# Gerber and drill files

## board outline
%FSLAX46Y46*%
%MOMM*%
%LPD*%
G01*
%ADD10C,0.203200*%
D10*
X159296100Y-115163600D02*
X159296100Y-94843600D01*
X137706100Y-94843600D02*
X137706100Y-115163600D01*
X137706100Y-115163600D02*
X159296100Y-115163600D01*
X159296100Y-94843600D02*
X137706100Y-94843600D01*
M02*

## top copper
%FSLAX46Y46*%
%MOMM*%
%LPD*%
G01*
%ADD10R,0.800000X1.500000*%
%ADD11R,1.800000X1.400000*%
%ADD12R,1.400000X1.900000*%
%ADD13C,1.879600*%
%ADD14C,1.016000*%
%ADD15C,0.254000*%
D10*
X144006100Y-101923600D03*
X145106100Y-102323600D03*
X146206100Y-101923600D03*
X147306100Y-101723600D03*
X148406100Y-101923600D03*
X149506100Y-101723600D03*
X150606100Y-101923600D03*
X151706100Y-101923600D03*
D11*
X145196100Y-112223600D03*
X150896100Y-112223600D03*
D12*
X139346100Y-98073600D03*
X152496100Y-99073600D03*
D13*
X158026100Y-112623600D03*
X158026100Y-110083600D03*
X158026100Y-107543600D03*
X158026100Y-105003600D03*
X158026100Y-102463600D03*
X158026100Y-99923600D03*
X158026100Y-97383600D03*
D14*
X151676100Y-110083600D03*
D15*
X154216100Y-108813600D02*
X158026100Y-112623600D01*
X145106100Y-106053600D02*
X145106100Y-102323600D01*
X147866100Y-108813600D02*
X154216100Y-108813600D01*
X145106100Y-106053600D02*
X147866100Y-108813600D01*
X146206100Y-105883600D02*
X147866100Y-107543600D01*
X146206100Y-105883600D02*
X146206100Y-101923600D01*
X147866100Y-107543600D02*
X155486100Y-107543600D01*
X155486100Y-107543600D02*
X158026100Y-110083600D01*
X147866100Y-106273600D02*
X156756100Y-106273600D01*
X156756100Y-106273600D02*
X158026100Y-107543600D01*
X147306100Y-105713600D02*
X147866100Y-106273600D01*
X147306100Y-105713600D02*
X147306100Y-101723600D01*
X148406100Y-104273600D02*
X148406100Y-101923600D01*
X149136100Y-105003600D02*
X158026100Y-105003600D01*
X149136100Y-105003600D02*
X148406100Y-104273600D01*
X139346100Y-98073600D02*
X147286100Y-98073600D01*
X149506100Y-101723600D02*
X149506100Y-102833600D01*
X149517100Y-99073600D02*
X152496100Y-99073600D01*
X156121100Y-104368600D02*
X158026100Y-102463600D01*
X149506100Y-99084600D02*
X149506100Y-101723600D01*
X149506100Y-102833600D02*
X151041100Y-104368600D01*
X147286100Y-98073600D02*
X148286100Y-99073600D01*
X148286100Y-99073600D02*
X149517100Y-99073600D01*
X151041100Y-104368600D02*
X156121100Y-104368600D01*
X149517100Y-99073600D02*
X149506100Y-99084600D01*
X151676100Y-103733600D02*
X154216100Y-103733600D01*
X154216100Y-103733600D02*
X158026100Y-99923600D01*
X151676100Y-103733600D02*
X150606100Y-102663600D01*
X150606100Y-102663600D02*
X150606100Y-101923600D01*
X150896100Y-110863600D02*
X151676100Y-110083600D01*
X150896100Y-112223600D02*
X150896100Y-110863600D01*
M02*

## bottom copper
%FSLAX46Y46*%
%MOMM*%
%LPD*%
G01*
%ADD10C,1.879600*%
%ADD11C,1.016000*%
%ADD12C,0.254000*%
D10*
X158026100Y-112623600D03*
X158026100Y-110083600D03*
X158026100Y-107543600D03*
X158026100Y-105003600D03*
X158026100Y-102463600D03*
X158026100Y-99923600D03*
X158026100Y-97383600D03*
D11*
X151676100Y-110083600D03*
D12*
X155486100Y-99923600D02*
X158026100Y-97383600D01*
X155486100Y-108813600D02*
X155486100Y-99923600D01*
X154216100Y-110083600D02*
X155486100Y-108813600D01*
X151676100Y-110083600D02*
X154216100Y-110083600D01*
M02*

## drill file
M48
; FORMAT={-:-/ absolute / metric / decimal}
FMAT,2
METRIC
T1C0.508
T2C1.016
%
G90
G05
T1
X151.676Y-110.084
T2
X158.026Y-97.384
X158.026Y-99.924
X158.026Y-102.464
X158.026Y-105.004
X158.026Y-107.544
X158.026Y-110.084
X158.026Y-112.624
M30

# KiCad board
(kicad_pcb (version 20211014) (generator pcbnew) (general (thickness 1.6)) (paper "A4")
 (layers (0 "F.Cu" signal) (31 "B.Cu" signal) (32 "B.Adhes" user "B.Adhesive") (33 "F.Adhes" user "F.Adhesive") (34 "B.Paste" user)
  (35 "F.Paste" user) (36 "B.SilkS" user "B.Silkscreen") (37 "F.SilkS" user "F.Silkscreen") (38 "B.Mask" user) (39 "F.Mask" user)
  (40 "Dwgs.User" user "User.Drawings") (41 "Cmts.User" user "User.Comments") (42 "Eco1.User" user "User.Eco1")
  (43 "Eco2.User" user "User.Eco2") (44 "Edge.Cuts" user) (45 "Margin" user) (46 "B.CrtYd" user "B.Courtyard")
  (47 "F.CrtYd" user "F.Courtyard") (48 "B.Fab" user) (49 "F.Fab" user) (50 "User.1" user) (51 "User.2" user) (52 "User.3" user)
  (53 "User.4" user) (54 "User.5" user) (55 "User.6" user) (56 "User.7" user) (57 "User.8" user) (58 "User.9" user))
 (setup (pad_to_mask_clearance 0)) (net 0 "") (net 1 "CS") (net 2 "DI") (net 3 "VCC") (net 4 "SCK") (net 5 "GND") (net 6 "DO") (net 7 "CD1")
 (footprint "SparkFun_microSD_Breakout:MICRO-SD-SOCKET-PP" (layer "F.Cu") (at 152.9461 112.6236)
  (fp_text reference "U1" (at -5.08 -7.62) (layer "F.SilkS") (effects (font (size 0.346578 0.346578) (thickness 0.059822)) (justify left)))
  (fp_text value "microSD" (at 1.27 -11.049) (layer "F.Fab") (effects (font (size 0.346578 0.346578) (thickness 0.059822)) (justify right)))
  (pad "1" smd rect (at -8.94 -10.7) (size 0.8 1.5) (layers "F.Cu" "F.Paste" "F.Mask") (solder_mask_margin 0.1016))
  (pad "2" smd rect (at -7.84 -10.3) (size 0.8 1.5) (layers "F.Cu" "F.Paste" "F.Mask") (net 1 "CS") (solder_mask_margin 0.1016))
  (pad "3" smd rect (at -6.74 -10.7) (size 0.8 1.5) (layers "F.Cu" "F.Paste" "F.Mask") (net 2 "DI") (solder_mask_margin 0.1016))
  (pad "4" smd rect (at -5.64 -10.9) (size 0.8 1.5) (layers "F.Cu" "F.Paste" "F.Mask") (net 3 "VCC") (solder_mask_margin 0.1016))
  (pad "5" smd rect (at -4.54 -10.7) (size 0.8 1.5) (layers "F.Cu" "F.Paste" "F.Mask") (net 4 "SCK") (solder_mask_margin 0.1016))
  (pad "6" smd rect (at -3.44 -10.9) (size 0.8 1.5) (layers "F.Cu" "F.Paste" "F.Mask") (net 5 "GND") (solder_mask_margin 0.1016))
  (pad "7" smd rect (at -2.34 -10.7) (size 0.8 1.5) (layers "F.Cu" "F.Paste" "F.Mask") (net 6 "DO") (solder_mask_margin 0.1016))
  (pad "8" smd rect (at -1.24 -10.7) (size 0.8 1.5) (layers "F.Cu" "F.Paste" "F.Mask") (solder_mask_margin 0.1016))
  (pad "CD1" smd rect (at -7.75 -0.4) (size 1.8 1.4) (layers "F.Cu" "F.Paste" "F.Mask") (solder_mask_margin 0.1016))
  (pad "CD2" smd rect (at -2.05 -0.4) (size 1.8 1.4) (layers "F.Cu" "F.Paste" "F.Mask") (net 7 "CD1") (solder_mask_margin 0.1016))
  (pad "GND1" smd rect (at -13.6 -14.55) (size 1.4 1.9) (layers "F.Cu" "F.Paste" "F.Mask") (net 5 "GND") (solder_mask_margin 0.1016))
  (pad "GND2" smd rect (at -0.45 -13.55) (size 1.4 1.9) (layers "F.Cu" "F.Paste" "F.Mask") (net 5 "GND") (solder_mask_margin 0.1016)))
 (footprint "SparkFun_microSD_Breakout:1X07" (layer "F.Cu") (at 158.0261 112.6236 90)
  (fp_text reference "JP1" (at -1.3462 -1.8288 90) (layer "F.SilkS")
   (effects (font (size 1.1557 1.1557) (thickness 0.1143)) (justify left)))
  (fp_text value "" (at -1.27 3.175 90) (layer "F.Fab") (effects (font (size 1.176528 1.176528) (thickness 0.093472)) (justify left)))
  (pad "1" thru_hole circle (at 0 0 180) (size 1.8796 1.8796) (drill 1.016) (layers *.Cu *.Mask) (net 1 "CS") (solder_mask_margin 0.1016))
  (pad "2" thru_hole circle (at 2.54 0 180) (size 1.8796 1.8796) (drill 1.016) (layers *.Cu *.Mask) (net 2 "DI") (solder_mask_margin 0.1016))
  (pad "3" thru_hole circle (at 5.08 0 180) (size 1.8796 1.8796) (drill 1.016) (layers *.Cu *.Mask) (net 3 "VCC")
   (solder_mask_margin 0.1016))
  (pad "4" thru_hole circle (at 7.62 0 180) (size 1.8796 1.8796) (drill 1.016) (layers *.Cu *.Mask) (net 4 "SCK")
   (solder_mask_margin 0.1016))
  (pad "5" thru_hole circle (at 10.16 0 180) (size 1.8796 1.8796) (drill 1.016) (layers *.Cu *.Mask) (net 5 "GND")
   (solder_mask_margin 0.1016))
  (pad "6" thru_hole circle (at 12.7 0 180) (size 1.8796 1.8796) (drill 1.016) (layers *.Cu *.Mask) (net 6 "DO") (solder_mask_margin 0.1016))
  (pad "7" thru_hole circle (at 15.24 0 180) (size 1.8796 1.8796) (drill 1.016) (layers *.Cu *.Mask) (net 7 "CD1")
   (solder_mask_margin 0.1016)))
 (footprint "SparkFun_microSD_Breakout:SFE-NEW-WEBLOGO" (layer "B.Cu") (at 155.8671 99.5426 -135)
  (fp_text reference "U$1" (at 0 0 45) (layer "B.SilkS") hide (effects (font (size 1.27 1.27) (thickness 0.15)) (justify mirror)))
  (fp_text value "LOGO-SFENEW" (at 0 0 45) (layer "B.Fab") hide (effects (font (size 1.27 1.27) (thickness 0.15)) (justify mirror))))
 (gr_line (start 159.2961 115.1636) (end 159.2961 94.8436) (layer "Edge.Cuts") (width 0.2032))
 (gr_line (start 137.7061 94.8436) (end 137.7061 115.1636) (layer "Edge.Cuts") (width 0.2032))
 (gr_line (start 137.7061 115.1636) (end 159.2961 115.1636) (layer "Edge.Cuts") (width 0.2032))
 (gr_line (start 159.2961 94.8436) (end 137.7061 94.8436) (layer "Edge.Cuts") (width 0.2032))
 (segment (start 154.2161 108.8136) (end 158.0261 112.6236) (width 0.254) (layer "F.Cu") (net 1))
 (segment (start 145.1061 106.0536) (end 145.1061 102.3236) (width 0.254) (layer "F.Cu") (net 1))
 (segment (start 147.8661 108.8136) (end 154.2161 108.8136) (width 0.254) (layer "F.Cu") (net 1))
 (segment (start 145.1061 106.0536) (end 147.8661 108.8136) (width 0.254) (layer "F.Cu") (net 1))
 (segment (start 146.2061 105.8836) (end 147.8661 107.5436) (width 0.254) (layer "F.Cu") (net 2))
 (segment (start 146.2061 105.8836) (end 146.2061 101.9236) (width 0.254) (layer "F.Cu") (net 2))
 (segment (start 147.8661 107.5436) (end 155.4861 107.5436) (width 0.254) (layer "F.Cu") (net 2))
 (segment (start 155.4861 107.5436) (end 158.0261 110.0836) (width 0.254) (layer "F.Cu") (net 2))
 (segment (start 147.8661 106.2736) (end 156.7561 106.2736) (width 0.254) (layer "F.Cu") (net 3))
 (segment (start 156.7561 106.2736) (end 158.0261 107.5436) (width 0.254) (layer "F.Cu") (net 3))
 (segment (start 147.3061 105.7136) (end 147.8661 106.2736) (width 0.254) (layer "F.Cu") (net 3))
 (segment (start 147.3061 105.7136) (end 147.3061 101.7236) (width 0.254) (layer "F.Cu") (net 3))
 (segment (start 148.4061 104.2736) (end 148.4061 101.9236) (width 0.254) (layer "F.Cu") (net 4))
 (segment (start 149.1361 105.0036) (end 158.0261 105.0036) (width 0.254) (layer "F.Cu") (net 4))
 (segment (start 149.1361 105.0036) (end 148.4061 104.2736) (width 0.254) (layer "F.Cu") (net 4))
 (segment (start 139.3461 98.0736) (end 147.2861 98.0736) (width 0.254) (layer "F.Cu") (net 5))
 (segment (start 149.5061 101.7236) (end 149.5061 102.8336) (width 0.254) (layer "F.Cu") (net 5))
 (segment (start 149.5171 99.0736) (end 152.4961 99.0736) (width 0.254) (layer "F.Cu") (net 5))
 (segment (start 156.1211 104.3686) (end 158.0261 102.4636) (width 0.254) (layer "F.Cu") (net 5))
 (segment (start 149.5061 99.0846) (end 149.5061 101.7236) (width 0.254) (layer "F.Cu") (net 5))
 (segment (start 149.5061 102.8336) (end 151.0411 104.3686) (width 0.254) (layer "F.Cu") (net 5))
 (segment (start 147.2861 98.0736) (end 148.2861 99.0736) (width 0.254) (layer "F.Cu") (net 5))
 (segment (start 148.2861 99.0736) (end 149.5171 99.0736) (width 0.254) (layer "F.Cu") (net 5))
 (segment (start 151.0411 104.3686) (end 156.1211 104.3686) (width 0.254) (layer "F.Cu") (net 5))
 (segment (start 149.5171 99.0736) (end 149.5061 99.0846) (width 0.254) (layer "F.Cu") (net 5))
 (segment (start 151.6761 103.7336) (end 154.2161 103.7336) (width 0.254) (layer "F.Cu") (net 6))
 (segment (start 154.2161 103.7336) (end 158.0261 99.9236) (width 0.254) (layer "F.Cu") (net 6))
 (segment (start 151.6761 103.7336) (end 150.6061 102.6636) (width 0.254) (layer "F.Cu") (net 6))
 (segment (start 150.6061 102.6636) (end 150.6061 101.9236) (width 0.254) (layer "F.Cu") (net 6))
 (segment (start 150.8961 110.8636) (end 151.6761 110.0836) (width 0.254) (layer "F.Cu") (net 7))
 (segment (start 150.8961 112.2236) (end 150.8961 110.8636) (width 0.254) (layer "F.Cu") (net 7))
 (via (at 151.6761 110.0836) (size 1.016) (drill 0.508) (layers "F.Cu" "B.Cu") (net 7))
 (segment (start 155.4861 99.9236) (end 158.0261 97.3836) (width 0.254) (layer "B.Cu") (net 7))
 (segment (start 155.4861 108.8136) (end 155.4861 99.9236) (width 0.254) (layer "B.Cu") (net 7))
 (segment (start 154.2161 110.0836) (end 155.4861 108.8136) (width 0.254) (layer "B.Cu") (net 7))
 (segment (start 151.6761 110.0836) (end 154.2161 110.0836) (width 0.254) (layer "B.Cu") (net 7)))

